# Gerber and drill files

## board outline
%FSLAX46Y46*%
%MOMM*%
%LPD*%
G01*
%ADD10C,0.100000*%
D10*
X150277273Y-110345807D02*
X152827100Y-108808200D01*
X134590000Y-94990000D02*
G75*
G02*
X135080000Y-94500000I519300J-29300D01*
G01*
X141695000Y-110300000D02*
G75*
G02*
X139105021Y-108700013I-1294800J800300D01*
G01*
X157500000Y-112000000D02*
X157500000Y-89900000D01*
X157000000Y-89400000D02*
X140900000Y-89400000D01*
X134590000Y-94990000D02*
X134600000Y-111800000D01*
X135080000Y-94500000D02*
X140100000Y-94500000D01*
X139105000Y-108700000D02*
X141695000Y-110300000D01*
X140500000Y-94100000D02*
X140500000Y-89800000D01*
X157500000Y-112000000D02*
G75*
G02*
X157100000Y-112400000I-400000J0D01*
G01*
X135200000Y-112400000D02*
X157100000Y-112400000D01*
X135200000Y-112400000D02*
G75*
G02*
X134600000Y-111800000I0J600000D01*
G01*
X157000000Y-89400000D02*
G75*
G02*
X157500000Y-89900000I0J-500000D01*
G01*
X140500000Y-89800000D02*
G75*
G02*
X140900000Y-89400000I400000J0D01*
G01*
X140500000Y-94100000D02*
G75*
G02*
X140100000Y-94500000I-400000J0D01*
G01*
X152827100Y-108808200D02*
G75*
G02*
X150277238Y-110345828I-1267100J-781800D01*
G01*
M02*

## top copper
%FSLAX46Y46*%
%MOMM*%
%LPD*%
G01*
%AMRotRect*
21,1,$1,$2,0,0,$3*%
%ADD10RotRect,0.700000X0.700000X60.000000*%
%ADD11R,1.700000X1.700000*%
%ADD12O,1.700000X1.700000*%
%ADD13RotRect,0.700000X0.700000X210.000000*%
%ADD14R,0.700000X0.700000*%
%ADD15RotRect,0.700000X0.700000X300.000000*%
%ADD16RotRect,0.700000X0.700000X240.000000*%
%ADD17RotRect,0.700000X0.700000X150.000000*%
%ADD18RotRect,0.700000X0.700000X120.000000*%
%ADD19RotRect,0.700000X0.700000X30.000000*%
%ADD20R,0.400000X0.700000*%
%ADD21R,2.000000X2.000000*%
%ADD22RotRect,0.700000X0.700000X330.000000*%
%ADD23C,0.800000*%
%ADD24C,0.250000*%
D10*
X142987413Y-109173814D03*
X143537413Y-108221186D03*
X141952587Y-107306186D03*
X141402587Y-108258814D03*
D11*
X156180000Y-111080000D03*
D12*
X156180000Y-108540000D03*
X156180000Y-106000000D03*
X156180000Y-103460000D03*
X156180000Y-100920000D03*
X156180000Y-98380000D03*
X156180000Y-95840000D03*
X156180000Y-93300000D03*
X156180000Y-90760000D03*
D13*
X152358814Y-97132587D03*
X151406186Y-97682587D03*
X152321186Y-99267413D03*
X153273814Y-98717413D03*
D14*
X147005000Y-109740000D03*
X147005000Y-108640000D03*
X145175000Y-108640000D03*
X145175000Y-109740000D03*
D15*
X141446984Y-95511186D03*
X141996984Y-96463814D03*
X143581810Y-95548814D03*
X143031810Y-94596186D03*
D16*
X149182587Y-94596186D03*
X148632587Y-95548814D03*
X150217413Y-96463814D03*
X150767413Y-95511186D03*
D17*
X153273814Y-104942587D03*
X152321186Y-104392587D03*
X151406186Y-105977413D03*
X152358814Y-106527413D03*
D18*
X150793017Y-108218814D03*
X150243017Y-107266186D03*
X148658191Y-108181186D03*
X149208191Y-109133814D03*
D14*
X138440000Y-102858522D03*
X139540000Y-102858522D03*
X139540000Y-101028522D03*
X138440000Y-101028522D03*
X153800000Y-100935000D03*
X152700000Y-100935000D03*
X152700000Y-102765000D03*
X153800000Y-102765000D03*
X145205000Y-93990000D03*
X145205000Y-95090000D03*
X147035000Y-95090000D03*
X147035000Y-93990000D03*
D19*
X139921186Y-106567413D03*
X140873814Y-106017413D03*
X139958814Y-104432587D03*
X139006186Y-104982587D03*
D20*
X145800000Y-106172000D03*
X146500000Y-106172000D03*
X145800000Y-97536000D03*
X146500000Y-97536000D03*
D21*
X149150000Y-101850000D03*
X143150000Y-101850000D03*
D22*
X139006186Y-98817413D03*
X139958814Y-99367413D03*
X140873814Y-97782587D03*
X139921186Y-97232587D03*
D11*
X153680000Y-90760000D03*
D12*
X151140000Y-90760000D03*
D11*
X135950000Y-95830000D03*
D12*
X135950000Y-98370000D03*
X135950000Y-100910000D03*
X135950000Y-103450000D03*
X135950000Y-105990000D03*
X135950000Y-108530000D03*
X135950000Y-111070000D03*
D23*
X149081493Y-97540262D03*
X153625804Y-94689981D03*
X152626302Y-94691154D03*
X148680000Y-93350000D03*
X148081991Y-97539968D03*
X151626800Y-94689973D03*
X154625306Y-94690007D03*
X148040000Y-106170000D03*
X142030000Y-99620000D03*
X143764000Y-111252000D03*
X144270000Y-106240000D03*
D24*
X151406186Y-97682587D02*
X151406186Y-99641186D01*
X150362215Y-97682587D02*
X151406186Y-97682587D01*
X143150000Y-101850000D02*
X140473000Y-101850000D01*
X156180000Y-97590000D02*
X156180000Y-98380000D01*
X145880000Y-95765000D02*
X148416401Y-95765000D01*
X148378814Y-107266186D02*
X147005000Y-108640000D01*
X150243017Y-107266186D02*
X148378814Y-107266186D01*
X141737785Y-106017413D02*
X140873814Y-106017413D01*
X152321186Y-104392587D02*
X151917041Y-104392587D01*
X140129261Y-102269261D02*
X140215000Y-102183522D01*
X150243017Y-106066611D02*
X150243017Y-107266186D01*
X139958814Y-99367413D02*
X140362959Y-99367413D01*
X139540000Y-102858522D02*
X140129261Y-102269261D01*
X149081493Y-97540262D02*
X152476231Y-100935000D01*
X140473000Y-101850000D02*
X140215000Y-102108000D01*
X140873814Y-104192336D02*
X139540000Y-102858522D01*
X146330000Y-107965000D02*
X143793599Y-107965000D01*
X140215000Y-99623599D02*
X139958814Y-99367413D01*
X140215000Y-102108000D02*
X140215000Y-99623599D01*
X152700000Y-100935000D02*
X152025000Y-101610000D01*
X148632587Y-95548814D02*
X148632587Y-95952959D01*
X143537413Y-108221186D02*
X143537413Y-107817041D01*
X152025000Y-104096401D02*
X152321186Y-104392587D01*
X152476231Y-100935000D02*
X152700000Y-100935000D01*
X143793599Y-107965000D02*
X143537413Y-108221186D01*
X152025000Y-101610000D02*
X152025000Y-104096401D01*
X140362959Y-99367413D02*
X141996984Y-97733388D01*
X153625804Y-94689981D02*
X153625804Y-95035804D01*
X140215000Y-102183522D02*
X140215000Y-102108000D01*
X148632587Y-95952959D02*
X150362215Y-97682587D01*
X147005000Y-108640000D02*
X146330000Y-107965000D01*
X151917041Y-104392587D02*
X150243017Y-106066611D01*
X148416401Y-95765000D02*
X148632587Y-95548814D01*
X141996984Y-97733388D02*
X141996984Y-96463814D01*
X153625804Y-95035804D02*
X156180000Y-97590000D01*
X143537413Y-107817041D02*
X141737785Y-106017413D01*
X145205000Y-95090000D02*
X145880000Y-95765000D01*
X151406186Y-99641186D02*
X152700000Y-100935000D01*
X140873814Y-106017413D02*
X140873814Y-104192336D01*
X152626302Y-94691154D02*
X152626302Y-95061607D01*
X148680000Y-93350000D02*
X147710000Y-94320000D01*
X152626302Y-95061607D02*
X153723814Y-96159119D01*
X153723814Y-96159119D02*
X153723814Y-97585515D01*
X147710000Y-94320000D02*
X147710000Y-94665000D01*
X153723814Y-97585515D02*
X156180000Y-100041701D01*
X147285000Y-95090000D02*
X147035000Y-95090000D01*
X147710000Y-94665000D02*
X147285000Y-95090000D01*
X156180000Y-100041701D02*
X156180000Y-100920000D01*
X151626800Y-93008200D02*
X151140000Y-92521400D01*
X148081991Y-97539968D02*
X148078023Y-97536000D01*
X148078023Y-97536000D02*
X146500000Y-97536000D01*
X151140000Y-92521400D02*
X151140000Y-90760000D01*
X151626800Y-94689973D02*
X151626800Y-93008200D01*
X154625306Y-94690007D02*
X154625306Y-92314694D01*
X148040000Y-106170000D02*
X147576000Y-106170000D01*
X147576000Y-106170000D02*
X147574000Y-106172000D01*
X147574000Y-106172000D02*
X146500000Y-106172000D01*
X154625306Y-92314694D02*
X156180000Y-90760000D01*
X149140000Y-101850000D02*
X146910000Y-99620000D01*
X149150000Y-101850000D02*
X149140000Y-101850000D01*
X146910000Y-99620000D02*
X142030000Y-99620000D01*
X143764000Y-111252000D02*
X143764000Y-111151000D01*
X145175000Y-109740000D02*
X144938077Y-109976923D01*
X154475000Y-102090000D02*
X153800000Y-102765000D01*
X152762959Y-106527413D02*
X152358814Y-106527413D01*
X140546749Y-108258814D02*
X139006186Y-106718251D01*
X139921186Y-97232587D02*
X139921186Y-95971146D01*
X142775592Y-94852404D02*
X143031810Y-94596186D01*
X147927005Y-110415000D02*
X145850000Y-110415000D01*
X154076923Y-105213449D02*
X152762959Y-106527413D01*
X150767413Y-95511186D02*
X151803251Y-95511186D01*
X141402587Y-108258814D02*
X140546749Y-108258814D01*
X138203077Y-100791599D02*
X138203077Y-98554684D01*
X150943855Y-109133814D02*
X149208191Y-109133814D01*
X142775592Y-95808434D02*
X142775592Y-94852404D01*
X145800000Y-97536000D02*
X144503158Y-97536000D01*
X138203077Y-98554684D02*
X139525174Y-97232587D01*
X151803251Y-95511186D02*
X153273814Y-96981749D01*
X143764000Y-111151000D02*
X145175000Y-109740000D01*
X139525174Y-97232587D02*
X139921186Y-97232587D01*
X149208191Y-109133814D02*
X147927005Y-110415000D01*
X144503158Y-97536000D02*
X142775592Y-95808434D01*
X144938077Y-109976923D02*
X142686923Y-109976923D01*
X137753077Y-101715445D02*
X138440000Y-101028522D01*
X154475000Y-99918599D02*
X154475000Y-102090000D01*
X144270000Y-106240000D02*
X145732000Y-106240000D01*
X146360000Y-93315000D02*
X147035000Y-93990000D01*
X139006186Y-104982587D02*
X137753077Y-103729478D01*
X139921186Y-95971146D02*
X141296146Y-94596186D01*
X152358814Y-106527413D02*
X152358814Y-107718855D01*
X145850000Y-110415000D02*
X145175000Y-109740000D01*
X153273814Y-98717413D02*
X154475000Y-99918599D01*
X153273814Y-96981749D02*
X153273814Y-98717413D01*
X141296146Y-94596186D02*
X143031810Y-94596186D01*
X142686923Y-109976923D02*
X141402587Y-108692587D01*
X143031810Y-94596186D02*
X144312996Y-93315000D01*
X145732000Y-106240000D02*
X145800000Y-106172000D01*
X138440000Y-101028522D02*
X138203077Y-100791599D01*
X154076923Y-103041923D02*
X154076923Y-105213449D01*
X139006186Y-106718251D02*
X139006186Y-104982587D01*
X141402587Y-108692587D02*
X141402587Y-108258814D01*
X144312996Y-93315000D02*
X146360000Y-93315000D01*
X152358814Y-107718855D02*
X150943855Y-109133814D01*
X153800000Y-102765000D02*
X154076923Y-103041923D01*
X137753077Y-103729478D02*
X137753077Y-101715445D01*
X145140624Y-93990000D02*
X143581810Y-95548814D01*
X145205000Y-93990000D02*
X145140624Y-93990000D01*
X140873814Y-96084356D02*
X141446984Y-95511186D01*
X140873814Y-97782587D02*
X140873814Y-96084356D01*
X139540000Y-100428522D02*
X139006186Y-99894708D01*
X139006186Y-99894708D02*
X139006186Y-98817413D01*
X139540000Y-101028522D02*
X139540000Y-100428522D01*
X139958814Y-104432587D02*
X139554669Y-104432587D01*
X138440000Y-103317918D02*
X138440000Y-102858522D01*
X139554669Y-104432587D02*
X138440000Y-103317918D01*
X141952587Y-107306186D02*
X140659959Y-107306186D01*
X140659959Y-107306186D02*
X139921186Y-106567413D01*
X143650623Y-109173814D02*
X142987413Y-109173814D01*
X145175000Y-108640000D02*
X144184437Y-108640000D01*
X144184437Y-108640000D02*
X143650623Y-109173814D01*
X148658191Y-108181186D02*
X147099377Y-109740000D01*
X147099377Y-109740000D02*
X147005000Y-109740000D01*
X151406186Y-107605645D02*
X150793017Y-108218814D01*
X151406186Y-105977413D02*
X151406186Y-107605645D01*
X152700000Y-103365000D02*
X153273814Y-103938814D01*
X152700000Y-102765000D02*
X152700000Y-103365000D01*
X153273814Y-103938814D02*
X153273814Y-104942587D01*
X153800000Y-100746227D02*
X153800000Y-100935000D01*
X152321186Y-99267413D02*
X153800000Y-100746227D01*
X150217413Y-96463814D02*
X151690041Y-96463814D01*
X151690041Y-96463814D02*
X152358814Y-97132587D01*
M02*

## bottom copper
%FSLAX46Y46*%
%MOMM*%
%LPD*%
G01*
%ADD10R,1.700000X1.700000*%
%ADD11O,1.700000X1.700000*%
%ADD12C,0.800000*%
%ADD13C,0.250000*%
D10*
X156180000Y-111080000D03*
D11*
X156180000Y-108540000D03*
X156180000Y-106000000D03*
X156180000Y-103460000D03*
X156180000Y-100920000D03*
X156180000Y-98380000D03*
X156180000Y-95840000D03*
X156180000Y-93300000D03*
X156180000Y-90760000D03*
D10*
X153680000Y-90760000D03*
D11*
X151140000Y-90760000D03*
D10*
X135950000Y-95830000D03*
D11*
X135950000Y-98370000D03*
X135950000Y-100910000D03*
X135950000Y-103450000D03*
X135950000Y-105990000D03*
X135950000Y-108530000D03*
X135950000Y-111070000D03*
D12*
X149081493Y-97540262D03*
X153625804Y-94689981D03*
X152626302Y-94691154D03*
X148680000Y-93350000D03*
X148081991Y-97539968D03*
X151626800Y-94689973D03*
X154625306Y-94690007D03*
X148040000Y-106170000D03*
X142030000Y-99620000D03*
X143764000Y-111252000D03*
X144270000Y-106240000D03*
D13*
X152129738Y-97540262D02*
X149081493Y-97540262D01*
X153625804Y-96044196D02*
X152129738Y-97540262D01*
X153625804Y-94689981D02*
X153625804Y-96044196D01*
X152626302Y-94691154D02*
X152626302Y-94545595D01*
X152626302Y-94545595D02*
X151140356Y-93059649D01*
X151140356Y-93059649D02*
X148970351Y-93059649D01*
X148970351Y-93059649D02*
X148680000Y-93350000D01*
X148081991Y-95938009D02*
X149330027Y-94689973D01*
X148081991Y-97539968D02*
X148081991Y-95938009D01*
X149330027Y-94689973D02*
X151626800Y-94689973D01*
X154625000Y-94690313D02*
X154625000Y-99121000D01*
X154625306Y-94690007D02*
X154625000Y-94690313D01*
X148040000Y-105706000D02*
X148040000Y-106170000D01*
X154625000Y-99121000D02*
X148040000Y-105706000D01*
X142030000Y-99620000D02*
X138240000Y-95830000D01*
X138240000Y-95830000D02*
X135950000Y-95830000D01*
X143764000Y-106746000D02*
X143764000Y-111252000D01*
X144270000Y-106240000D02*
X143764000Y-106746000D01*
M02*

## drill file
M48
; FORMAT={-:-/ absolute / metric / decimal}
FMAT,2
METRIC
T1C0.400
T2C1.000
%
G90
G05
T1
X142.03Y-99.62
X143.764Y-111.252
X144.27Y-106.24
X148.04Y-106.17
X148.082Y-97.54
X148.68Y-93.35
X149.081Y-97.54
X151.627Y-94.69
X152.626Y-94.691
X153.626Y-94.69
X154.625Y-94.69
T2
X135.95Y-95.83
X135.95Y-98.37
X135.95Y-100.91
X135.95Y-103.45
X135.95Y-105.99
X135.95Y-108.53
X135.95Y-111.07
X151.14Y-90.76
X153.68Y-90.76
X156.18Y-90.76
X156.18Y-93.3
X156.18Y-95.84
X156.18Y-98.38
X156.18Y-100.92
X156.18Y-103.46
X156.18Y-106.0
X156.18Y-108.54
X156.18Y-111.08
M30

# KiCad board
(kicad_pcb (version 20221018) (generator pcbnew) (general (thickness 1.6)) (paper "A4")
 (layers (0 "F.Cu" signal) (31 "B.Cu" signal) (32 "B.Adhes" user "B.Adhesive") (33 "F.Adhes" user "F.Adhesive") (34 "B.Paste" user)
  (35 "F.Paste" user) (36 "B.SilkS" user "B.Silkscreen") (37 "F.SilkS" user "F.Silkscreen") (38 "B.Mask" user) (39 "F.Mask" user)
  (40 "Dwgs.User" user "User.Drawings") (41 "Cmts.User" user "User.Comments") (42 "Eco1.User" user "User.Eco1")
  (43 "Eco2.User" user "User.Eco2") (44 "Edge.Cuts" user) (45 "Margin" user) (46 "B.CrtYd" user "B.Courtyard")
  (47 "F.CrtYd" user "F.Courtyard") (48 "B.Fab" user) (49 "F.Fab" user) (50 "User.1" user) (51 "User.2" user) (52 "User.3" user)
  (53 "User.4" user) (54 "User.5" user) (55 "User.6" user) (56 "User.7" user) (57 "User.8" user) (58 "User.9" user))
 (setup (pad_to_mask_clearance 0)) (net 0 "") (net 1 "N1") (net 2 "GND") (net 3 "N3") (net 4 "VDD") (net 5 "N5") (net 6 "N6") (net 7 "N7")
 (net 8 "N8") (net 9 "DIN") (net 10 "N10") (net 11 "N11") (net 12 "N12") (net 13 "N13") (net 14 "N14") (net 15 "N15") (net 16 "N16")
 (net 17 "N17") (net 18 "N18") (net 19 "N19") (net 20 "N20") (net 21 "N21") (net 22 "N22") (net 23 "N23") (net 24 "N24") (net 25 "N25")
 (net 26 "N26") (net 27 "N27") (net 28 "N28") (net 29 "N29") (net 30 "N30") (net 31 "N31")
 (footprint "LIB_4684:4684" (layer "F.Cu") (at 142.47 108.24 -30)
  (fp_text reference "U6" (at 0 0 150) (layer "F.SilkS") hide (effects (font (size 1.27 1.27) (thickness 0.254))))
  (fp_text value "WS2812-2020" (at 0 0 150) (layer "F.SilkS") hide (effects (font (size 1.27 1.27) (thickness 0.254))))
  (pad "1" smd rect (at 0.915 0.55 60) (size 0.7 0.7) (layers "F.Cu" "F.Paste" "F.Mask") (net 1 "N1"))
  (pad "2" smd rect (at 0.915 -0.55 60) (size 0.7 0.7) (layers "F.Cu" "F.Paste" "F.Mask") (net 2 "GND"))
  (pad "3" smd rect (at -0.915 -0.55 60) (size 0.7 0.7) (layers "F.Cu" "F.Paste" "F.Mask") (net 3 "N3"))
  (pad "4" smd rect (at -0.915 0.55 60) (size 0.7 0.7) (layers "F.Cu" "F.Paste" "F.Mask") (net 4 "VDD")))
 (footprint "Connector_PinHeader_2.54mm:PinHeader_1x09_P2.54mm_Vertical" (layer "F.Cu") (at 156.18 111.08 180)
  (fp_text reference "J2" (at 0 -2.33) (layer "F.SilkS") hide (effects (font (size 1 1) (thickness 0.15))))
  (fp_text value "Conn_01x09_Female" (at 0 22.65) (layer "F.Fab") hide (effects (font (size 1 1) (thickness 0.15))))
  (pad "1" thru_hole rect (at 0 0 180) (size 1.7 1.7) (drill 1) (layers "*.Cu" "*.Mask") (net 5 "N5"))
  (pad "2" thru_hole oval (at 0 2.54 180) (size 1.7 1.7) (drill 1) (layers "*.Cu" "*.Mask") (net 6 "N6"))
  (pad "3" thru_hole oval (at 0 5.08 180) (size 1.7 1.7) (drill 1) (layers "*.Cu" "*.Mask") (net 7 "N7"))
  (pad "4" thru_hole oval (at 0 7.62 180) (size 1.7 1.7) (drill 1) (layers "*.Cu" "*.Mask") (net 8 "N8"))
  (pad "5" thru_hole oval (at 0 10.16 180) (size 1.7 1.7) (drill 1) (layers "*.Cu" "*.Mask") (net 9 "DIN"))
  (pad "6" thru_hole oval (at 0 12.7 180) (size 1.7 1.7) (drill 1) (layers "*.Cu" "*.Mask") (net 2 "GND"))
  (pad "7" thru_hole oval (at 0 15.24 180) (size 1.7 1.7) (drill 1) (layers "*.Cu" "*.Mask") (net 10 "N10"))
  (pad "8" thru_hole oval (at 0 17.78 180) (size 1.7 1.7) (drill 1) (layers "*.Cu" "*.Mask") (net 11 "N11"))
  (pad "9" thru_hole oval (at 0 20.32 180) (size 1.7 1.7) (drill 1) (layers "*.Cu" "*.Mask") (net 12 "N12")))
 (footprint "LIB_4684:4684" (layer "F.Cu") (at 152.34 98.2 120)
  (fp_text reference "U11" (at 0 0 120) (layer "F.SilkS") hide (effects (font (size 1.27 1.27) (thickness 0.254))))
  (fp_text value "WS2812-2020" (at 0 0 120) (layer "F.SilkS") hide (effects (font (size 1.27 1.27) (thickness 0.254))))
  (pad "1" smd rect (at 0.915 0.55 210) (size 0.7 0.7) (layers "F.Cu" "F.Paste" "F.Mask") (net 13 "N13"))
  (pad "2" smd rect (at 0.915 -0.55 210) (size 0.7 0.7) (layers "F.Cu" "F.Paste" "F.Mask") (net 2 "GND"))
  (pad "3" smd rect (at -0.915 -0.55 210) (size 0.7 0.7) (layers "F.Cu" "F.Paste" "F.Mask") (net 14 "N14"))
  (pad "4" smd rect (at -0.915 0.55 210) (size 0.7 0.7) (layers "F.Cu" "F.Paste" "F.Mask") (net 4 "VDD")))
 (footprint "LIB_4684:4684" (layer "F.Cu") (at 146.09 109.19)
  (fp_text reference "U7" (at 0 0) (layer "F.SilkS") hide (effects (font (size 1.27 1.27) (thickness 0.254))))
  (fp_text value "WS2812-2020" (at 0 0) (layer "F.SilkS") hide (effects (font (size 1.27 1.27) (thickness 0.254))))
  (pad "1" smd rect (at 0.915 0.55 90) (size 0.7 0.7) (layers "F.Cu" "F.Paste" "F.Mask") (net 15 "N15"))
  (pad "2" smd rect (at 0.915 -0.55 90) (size 0.7 0.7) (layers "F.Cu" "F.Paste" "F.Mask") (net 2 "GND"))
  (pad "3" smd rect (at -0.915 -0.55 90) (size 0.7 0.7) (layers "F.Cu" "F.Paste" "F.Mask") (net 1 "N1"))
  (pad "4" smd rect (at -0.915 0.55 90) (size 0.7 0.7) (layers "F.Cu" "F.Paste" "F.Mask") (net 4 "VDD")))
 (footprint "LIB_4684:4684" (layer "F.Cu") (at 142.514397 95.53 -150)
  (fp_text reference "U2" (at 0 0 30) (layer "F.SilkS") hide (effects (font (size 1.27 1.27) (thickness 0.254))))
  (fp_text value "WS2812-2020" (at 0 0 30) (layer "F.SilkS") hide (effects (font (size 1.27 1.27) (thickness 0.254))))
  (pad "1" smd rect (at 0.915 0.55 300) (size 0.7 0.7) (layers "F.Cu" "F.Paste" "F.Mask") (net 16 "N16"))
  (pad "2" smd rect (at 0.915 -0.55 300) (size 0.7 0.7) (layers "F.Cu" "F.Paste" "F.Mask") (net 2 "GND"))
  (pad "3" smd rect (at -0.915 -0.55 300) (size 0.7 0.7) (layers "F.Cu" "F.Paste" "F.Mask") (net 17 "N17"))
  (pad "4" smd rect (at -0.915 0.55 300) (size 0.7 0.7) (layers "F.Cu" "F.Paste" "F.Mask") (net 4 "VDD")))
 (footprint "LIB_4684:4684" (layer "F.Cu") (at 149.7 95.53 150)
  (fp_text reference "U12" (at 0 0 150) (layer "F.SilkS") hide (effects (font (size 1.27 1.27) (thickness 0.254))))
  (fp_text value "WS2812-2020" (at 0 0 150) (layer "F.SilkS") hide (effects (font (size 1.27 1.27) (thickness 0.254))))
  (pad "1" smd rect (at 0.915 0.55 240) (size 0.7 0.7) (layers "F.Cu" "F.Paste" "F.Mask") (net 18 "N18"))
  (pad "2" smd rect (at 0.915 -0.55 240) (size 0.7 0.7) (layers "F.Cu" "F.Paste" "F.Mask") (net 2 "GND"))
  (pad "3" smd rect (at -0.915 -0.55 240) (size 0.7 0.7) (layers "F.Cu" "F.Paste" "F.Mask") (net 13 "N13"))
  (pad "4" smd rect (at -0.915 0.55 240) (size 0.7 0.7) (layers "F.Cu" "F.Paste" "F.Mask") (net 4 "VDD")))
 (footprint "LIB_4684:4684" (layer "F.Cu") (at 152.34 105.46 60)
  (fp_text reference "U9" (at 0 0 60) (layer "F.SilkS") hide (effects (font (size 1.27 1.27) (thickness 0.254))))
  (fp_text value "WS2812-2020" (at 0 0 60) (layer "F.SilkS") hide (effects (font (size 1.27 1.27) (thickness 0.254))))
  (pad "1" smd rect (at 0.915 0.55 150) (size 0.7 0.7) (layers "F.Cu" "F.Paste" "F.Mask") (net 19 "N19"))
  (pad "2" smd rect (at 0.915 -0.55 150) (size 0.7 0.7) (layers "F.Cu" "F.Paste" "F.Mask") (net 2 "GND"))
  (pad "3" smd rect (at -0.915 -0.55 150) (size 0.7 0.7) (layers "F.Cu" "F.Paste" "F.Mask") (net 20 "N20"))
  (pad "4" smd rect (at -0.915 0.55 150) (size 0.7 0.7) (layers "F.Cu" "F.Paste" "F.Mask") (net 4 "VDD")))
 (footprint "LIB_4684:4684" (layer "F.Cu") (at 149.725604 108.2 30)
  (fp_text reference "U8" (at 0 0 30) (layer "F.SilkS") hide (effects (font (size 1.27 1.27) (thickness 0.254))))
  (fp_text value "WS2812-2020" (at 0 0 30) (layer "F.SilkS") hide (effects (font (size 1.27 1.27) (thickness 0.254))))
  (pad "1" smd rect (at 0.915 0.55 120) (size 0.7 0.7) (layers "F.Cu" "F.Paste" "F.Mask") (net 20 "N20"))
  (pad "2" smd rect (at 0.915 -0.55 120) (size 0.7 0.7) (layers "F.Cu" "F.Paste" "F.Mask") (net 2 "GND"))
  (pad "3" smd rect (at -0.915 -0.55 120) (size 0.7 0.7) (layers "F.Cu" "F.Paste" "F.Mask") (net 15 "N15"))
  (pad "4" smd rect (at -0.915 0.55 120) (size 0.7 0.7) (layers "F.Cu" "F.Paste" "F.Mask") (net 4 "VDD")))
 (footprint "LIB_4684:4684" (layer "F.Cu") (at 138.99 101.943522 -90)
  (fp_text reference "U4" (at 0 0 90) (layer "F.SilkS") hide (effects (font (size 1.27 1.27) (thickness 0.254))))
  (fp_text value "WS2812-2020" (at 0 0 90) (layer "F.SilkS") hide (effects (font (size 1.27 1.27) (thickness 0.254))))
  (pad "1" smd rect (at 0.915 0.55) (size 0.7 0.7) (layers "F.Cu" "F.Paste" "F.Mask") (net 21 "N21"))
  (pad "2" smd rect (at 0.915 -0.55) (size 0.7 0.7) (layers "F.Cu" "F.Paste" "F.Mask") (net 2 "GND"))
  (pad "3" smd rect (at -0.915 -0.55) (size 0.7 0.7) (layers "F.Cu" "F.Paste" "F.Mask") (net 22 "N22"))
  (pad "4" smd rect (at -0.915 0.55) (size 0.7 0.7) (layers "F.Cu" "F.Paste" "F.Mask") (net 4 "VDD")))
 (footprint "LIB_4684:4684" (layer "F.Cu") (at 153.25 101.85 90)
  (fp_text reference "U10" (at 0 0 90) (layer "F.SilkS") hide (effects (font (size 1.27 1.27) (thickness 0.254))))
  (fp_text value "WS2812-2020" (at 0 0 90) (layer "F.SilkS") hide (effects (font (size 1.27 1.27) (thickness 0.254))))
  (pad "1" smd rect (at 0.915 0.55 180) (size 0.7 0.7) (layers "F.Cu" "F.Paste" "F.Mask") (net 14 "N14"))
  (pad "2" smd rect (at 0.915 -0.55 180) (size 0.7 0.7) (layers "F.Cu" "F.Paste" "F.Mask") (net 2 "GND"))
  (pad "3" smd rect (at -0.915 -0.55 180) (size 0.7 0.7) (layers "F.Cu" "F.Paste" "F.Mask") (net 19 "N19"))
  (pad "4" smd rect (at -0.915 0.55 180) (size 0.7 0.7) (layers "F.Cu" "F.Paste" "F.Mask") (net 4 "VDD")))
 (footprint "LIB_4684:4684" (layer "F.Cu") (at 146.12 94.54 180)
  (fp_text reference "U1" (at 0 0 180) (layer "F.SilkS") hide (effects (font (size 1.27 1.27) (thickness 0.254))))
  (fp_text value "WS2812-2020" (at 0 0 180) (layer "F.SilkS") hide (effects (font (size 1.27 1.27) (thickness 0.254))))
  (pad "1" smd rect (at 0.915 0.55 270) (size 0.7 0.7) (layers "F.Cu" "F.Paste" "F.Mask") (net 17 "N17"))
  (pad "2" smd rect (at 0.915 -0.55 270) (size 0.7 0.7) (layers "F.Cu" "F.Paste" "F.Mask") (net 2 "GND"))
  (pad "3" smd rect (at -0.915 -0.55 270) (size 0.7 0.7) (layers "F.Cu" "F.Paste" "F.Mask") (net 9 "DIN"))
  (pad "4" smd rect (at -0.915 0.55 270) (size 0.7 0.7) (layers "F.Cu" "F.Paste" "F.Mask") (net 4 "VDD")))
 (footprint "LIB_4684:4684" (layer "F.Cu") (at 139.94 105.5 -60)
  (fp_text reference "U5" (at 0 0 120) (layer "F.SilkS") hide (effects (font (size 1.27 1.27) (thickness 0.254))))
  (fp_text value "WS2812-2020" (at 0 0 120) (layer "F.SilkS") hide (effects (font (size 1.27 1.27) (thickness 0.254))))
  (pad "1" smd rect (at 0.915 0.55 30) (size 0.7 0.7) (layers "F.Cu" "F.Paste" "F.Mask") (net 3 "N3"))
  (pad "2" smd rect (at 0.915 -0.55 30) (size 0.7 0.7) (layers "F.Cu" "F.Paste" "F.Mask") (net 2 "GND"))
  (pad "3" smd rect (at -0.915 -0.55 30) (size 0.7 0.7) (layers "F.Cu" "F.Paste" "F.Mask") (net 21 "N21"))
  (pad "4" smd rect (at -0.915 0.55 30) (size 0.7 0.7) (layers "F.Cu" "F.Paste" "F.Mask") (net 4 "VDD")))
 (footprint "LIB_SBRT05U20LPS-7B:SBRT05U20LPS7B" (layer "F.Cu") (at 146.15 106.172)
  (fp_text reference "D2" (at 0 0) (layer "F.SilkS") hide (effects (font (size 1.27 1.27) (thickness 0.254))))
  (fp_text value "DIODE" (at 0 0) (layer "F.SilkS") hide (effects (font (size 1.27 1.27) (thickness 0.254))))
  (pad "1" smd rect (at -0.35 0) (size 0.4 0.7) (layers "F.Cu" "F.Paste" "F.Mask") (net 4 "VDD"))
  (pad "2" smd rect (at 0.35 0) (size 0.4 0.7) (layers "F.Cu" "F.Paste" "F.Mask") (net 12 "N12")))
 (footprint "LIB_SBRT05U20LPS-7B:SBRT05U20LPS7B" (layer "F.Cu") (at 146.15 97.536)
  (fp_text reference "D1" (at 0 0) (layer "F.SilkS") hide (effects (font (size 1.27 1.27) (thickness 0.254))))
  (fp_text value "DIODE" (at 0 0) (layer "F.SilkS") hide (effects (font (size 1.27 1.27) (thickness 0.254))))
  (pad "1" smd rect (at -0.35 0) (size 0.4 0.7) (layers "F.Cu" "F.Paste" "F.Mask") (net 4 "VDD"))
  (pad "2" smd rect (at 0.35 0) (size 0.4 0.7) (layers "F.Cu" "F.Paste" "F.Mask") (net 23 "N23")))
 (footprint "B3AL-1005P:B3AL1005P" (layer "F.Cu") (at 146.15 101.85)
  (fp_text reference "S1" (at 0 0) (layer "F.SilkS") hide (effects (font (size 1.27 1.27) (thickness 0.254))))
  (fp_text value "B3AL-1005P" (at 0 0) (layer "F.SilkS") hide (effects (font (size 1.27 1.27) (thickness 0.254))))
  (pad "1" smd rect (at 3 0 90) (size 2 2) (layers "F.Cu" "F.Paste" "F.Mask") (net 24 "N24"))
  (pad "2" smd rect (at -3 0 90) (size 2 2) (layers "F.Cu" "F.Paste" "F.Mask") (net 2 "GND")))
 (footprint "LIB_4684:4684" (layer "F.Cu") (at 139.94 98.3 -120)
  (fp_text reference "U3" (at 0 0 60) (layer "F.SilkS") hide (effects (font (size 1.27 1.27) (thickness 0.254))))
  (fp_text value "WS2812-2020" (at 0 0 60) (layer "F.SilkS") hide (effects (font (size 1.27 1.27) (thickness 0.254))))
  (pad "1" smd rect (at 0.915 0.55 330) (size 0.7 0.7) (layers "F.Cu" "F.Paste" "F.Mask") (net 22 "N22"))
  (pad "2" smd rect (at 0.915 -0.55 330) (size 0.7 0.7) (layers "F.Cu" "F.Paste" "F.Mask") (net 2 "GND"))
  (pad "3" smd rect (at -0.915 -0.55 330) (size 0.7 0.7) (layers "F.Cu" "F.Paste" "F.Mask") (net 16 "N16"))
  (pad "4" smd rect (at -0.915 0.55 330) (size 0.7 0.7) (layers "F.Cu" "F.Paste" "F.Mask") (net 4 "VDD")))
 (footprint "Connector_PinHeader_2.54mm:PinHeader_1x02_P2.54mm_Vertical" (layer "F.Cu") (at 153.68 90.76 -90)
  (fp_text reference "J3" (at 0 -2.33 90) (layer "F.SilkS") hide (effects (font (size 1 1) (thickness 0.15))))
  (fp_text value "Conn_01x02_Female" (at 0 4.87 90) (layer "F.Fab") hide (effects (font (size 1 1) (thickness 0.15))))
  (pad "1" thru_hole rect (at 0 0 270) (size 1.7 1.7) (drill 1) (layers "*.Cu" "*.Mask") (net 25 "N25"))
  (pad "2" thru_hole oval (at 0 2.54 270) (size 1.7 1.7) (drill 1) (layers "*.Cu" "*.Mask") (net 23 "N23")))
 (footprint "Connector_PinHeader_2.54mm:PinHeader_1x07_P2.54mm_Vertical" (layer "F.Cu") (at 135.95 95.83)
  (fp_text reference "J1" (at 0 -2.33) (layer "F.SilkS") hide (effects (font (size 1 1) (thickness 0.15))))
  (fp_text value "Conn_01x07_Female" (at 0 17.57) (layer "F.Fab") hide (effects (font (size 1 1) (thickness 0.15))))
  (pad "1" thru_hole rect (at 0 0) (size 1.7 1.7) (drill 1) (layers "*.Cu" "*.Mask") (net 24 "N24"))
  (pad "2" thru_hole oval (at 0 2.54) (size 1.7 1.7) (drill 1) (layers "*.Cu" "*.Mask") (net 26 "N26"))
  (pad "3" thru_hole oval (at 0 5.08) (size 1.7 1.7) (drill 1) (layers "*.Cu" "*.Mask") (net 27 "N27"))
  (pad "4" thru_hole oval (at 0 7.62) (size 1.7 1.7) (drill 1) (layers "*.Cu" "*.Mask") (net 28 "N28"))
  (pad "5" thru_hole oval (at 0 10.16) (size 1.7 1.7) (drill 1) (layers "*.Cu" "*.Mask") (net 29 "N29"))
  (pad "6" thru_hole oval (at 0 12.7) (size 1.7 1.7) (drill 1) (layers "*.Cu" "*.Mask") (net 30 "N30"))
  (pad "7" thru_hole oval (at 0 15.24) (size 1.7 1.7) (drill 1) (layers "*.Cu" "*.Mask") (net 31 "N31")))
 (gr_line (start 150.277273 110.345807) (end 152.8271 108.8082) (stroke (width 0.1) (type solid)) (layer "Edge.Cuts"))
 (gr_arc (start 134.59 94.99) (mid 134.741518 94.651518) (end 135.08 94.5) (stroke (width 0.1) (type solid)) (layer "Edge.Cuts"))
 (gr_arc (start 141.695 110.3) (mid 139.600179 110.794634) (end 139.105 108.7) (stroke (width 0.1) (type solid)) (layer "Edge.Cuts"))
 (gr_line (start 157.5 112) (end 157.5 89.9) (stroke (width 0.1) (type solid)) (layer "Edge.Cuts"))
 (gr_line (start 157 89.4) (end 140.9 89.4) (stroke (width 0.1) (type solid)) (layer "Edge.Cuts"))
 (gr_line (start 134.59 94.99) (end 134.6 111.8) (stroke (width 0.1) (type solid)) (layer "Edge.Cuts"))
 (gr_line (start 135.08 94.5) (end 140.1 94.5) (stroke (width 0.1) (type solid)) (layer "Edge.Cuts"))
 (gr_line (start 139.105 108.7) (end 141.695 110.3) (stroke (width 0.1) (type solid)) (layer "Edge.Cuts"))
 (gr_line (start 140.5 94.1) (end 140.5 89.8) (stroke (width 0.1) (type solid)) (layer "Edge.Cuts"))
 (gr_arc (start 157.5 112) (mid 157.382843 112.282843) (end 157.1 112.4) (stroke (width 0.1) (type solid)) (layer "Edge.Cuts"))
 (gr_line (start 135.2 112.4) (end 157.1 112.4) (stroke (width 0.1) (type solid)) (layer "Edge.Cuts"))
 (gr_arc (start 135.2 112.4) (mid 134.775736 112.224264) (end 134.6 111.8) (stroke (width 0.1) (type solid)) (layer "Edge.Cuts"))
 (gr_arc (start 157 89.4) (mid 157.353553 89.546447) (end 157.5 89.9) (stroke (width 0.1) (type solid)) (layer "Edge.Cuts"))
 (gr_arc (start 140.5 89.8) (mid 140.617157 89.517157) (end 140.9 89.4) (stroke (width 0.1) (type solid)) (layer "Edge.Cuts"))
 (gr_arc (start 140.5 94.1) (mid 140.382843 94.382843) (end 140.1 94.5) (stroke (width 0.1) (type solid)) (layer "Edge.Cuts"))
 (gr_arc (start 152.8271 108.8082) (mid 152.328854 110.864997) (end 150.277273 110.345807) (stroke (width 0.1) (type solid))
  (layer "Edge.Cuts"))
 (segment (start 151.406186 97.682587) (end 151.406186 99.641186) (width 0.25) (layer "F.Cu") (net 2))
 (segment (start 150.362215 97.682587) (end 151.406186 97.682587) (width 0.25) (layer "F.Cu") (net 2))
 (segment (start 143.15 101.85) (end 140.473 101.85) (width 0.25) (layer "F.Cu") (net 2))
 (segment (start 156.18 97.59) (end 156.18 98.38) (width 0.25) (layer "F.Cu") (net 2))
 (segment (start 145.88 95.765) (end 148.416401 95.765) (width 0.25) (layer "F.Cu") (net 2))
 (segment (start 148.378814 107.266186) (end 147.005 108.64) (width 0.25) (layer "F.Cu") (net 2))
 (segment (start 150.243017 107.266186) (end 148.378814 107.266186) (width 0.25) (layer "F.Cu") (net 2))
 (segment (start 141.737785 106.017413) (end 140.873814 106.017413) (width 0.25) (layer "F.Cu") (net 2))
 (segment (start 152.321186 104.392587) (end 151.917041 104.392587) (width 0.25) (layer "F.Cu") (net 2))
 (segment (start 140.129261 102.269261) (end 140.215 102.183522) (width 0.25) (layer "F.Cu") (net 2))
 (segment (start 150.243017 106.066611) (end 150.243017 107.266186) (width 0.25) (layer "F.Cu") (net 2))
 (segment (start 139.958814 99.367413) (end 140.362959 99.367413) (width 0.25) (layer "F.Cu") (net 2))
 (segment (start 139.54 102.858522) (end 140.129261 102.269261) (width 0.25) (layer "F.Cu") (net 2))
 (segment (start 149.081493 97.540262) (end 152.476231 100.935) (width 0.25) (layer "F.Cu") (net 2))
 (segment (start 140.473 101.85) (end 140.215 102.108) (width 0.25) (layer "F.Cu") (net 2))
 (segment (start 140.873814 104.192336) (end 139.54 102.858522) (width 0.25) (layer "F.Cu") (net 2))
 (segment (start 146.33 107.965) (end 143.793599 107.965) (width 0.25) (layer "F.Cu") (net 2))
 (segment (start 140.215 99.623599) (end 139.958814 99.367413) (width 0.25) (layer "F.Cu") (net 2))
 (segment (start 140.215 102.108) (end 140.215 99.623599) (width 0.25) (layer "F.Cu") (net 2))
 (segment (start 152.7 100.935) (end 152.025 101.61) (width 0.25) (layer "F.Cu") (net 2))
 (segment (start 148.632587 95.548814) (end 148.632587 95.952959) (width 0.25) (layer "F.Cu") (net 2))
 (segment (start 143.537413 108.221186) (end 143.537413 107.817041) (width 0.25) (layer "F.Cu") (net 2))
 (segment (start 152.025 104.096401) (end 152.321186 104.392587) (width 0.25) (layer "F.Cu") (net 2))
 (segment (start 152.476231 100.935) (end 152.7 100.935) (width 0.25) (layer "F.Cu") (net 2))
 (segment (start 143.793599 107.965) (end 143.537413 108.221186) (width 0.25) (layer "F.Cu") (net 2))
 (segment (start 152.025 101.61) (end 152.025 104.096401) (width 0.25) (layer "F.Cu") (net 2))
 (segment (start 140.362959 99.367413) (end 141.996984 97.733388) (width 0.25) (layer "F.Cu") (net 2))
 (segment (start 153.625804 94.689981) (end 153.625804 95.035804) (width 0.25) (layer "F.Cu") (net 2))
 (segment (start 140.215 102.183522) (end 140.215 102.108) (width 0.25) (layer "F.Cu") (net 2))
 (segment (start 148.632587 95.952959) (end 150.362215 97.682587) (width 0.25) (layer "F.Cu") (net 2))
 (segment (start 147.005 108.64) (end 146.33 107.965) (width 0.25) (layer "F.Cu") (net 2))
 (segment (start 151.917041 104.392587) (end 150.243017 106.066611) (width 0.25) (layer "F.Cu") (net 2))
 (segment (start 148.416401 95.765) (end 148.632587 95.548814) (width 0.25) (layer "F.Cu") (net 2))
 (segment (start 141.996984 97.733388) (end 141.996984 96.463814) (width 0.25) (layer "F.Cu") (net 2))
 (segment (start 153.625804 95.035804) (end 156.18 97.59) (width 0.25) (layer "F.Cu") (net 2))
 (segment (start 143.537413 107.817041) (end 141.737785 106.017413) (width 0.25) (layer "F.Cu") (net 2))
 (segment (start 145.205 95.09) (end 145.88 95.765) (width 0.25) (layer "F.Cu") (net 2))
 (segment (start 151.406186 99.641186) (end 152.7 100.935) (width 0.25) (layer "F.Cu") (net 2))
 (segment (start 140.873814 106.017413) (end 140.873814 104.192336) (width 0.25) (layer "F.Cu") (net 2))
 (via (at 149.081493 97.540262) (size 0.8) (drill 0.4) (layers "F.Cu" "B.Cu") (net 2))
 (via (at 153.625804 94.689981) (size 0.8) (drill 0.4) (layers "F.Cu" "B.Cu") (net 2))
 (segment (start 152.129738 97.540262) (end 149.081493 97.540262) (width 0.25) (layer "B.Cu") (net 2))
 (segment (start 153.625804 96.044196) (end 152.129738 97.540262) (width 0.25) (layer "B.Cu") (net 2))
 (segment (start 153.625804 94.689981) (end 153.625804 96.044196) (width 0.25) (layer "B.Cu") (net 2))
 (segment (start 152.626302 94.691154) (end 152.626302 95.061607) (width 0.25) (layer "F.Cu") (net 9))
 (segment (start 148.68 93.35) (end 147.71 94.32) (width 0.25) (layer "F.Cu") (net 9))
 (segment (start 152.626302 95.061607) (end 153.723814 96.159119) (width 0.25) (layer "F.Cu") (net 9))
 (segment (start 153.723814 96.159119) (end 153.723814 97.585515) (width 0.25) (layer "F.Cu") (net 9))
 (segment (start 147.71 94.32) (end 147.71 94.665) (width 0.25) (layer "F.Cu") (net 9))
 (segment (start 153.723814 97.585515) (end 156.18 100.041701) (width 0.25) (layer "F.Cu") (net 9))
 (segment (start 147.285 95.09) (end 147.035 95.09) (width 0.25) (layer "F.Cu") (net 9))
 (segment (start 147.71 94.665) (end 147.285 95.09) (width 0.25) (layer "F.Cu") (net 9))
 (segment (start 156.18 100.041701) (end 156.18 100.92) (width 0.25) (layer "F.Cu") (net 9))
 (via (at 152.626302 94.691154) (size 0.8) (drill 0.4) (layers "F.Cu" "B.Cu") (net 9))
 (via (at 148.68 93.35) (size 0.8) (drill 0.4) (layers "F.Cu" "B.Cu") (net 9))
 (segment (start 152.626302 94.691154) (end 152.626302 94.545595) (width 0.25) (layer "B.Cu") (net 9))
 (segment (start 152.626302 94.545595) (end 151.140356 93.059649) (width 0.25) (layer "B.Cu") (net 9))
 (segment (start 151.140356 93.059649) (end 148.970351 93.059649) (width 0.25) (layer "B.Cu") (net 9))
 (segment (start 148.970351 93.059649) (end 148.68 93.35) (width 0.25) (layer "B.Cu") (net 9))
 (segment (start 151.6268 93.0082) (end 151.14 92.5214) (width 0.25) (layer "F.Cu") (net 23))
 (segment (start 148.081991 97.539968) (end 148.078023 97.536) (width 0.25) (layer "F.Cu") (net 23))
 (segment (start 148.078023 97.536) (end 146.5 97.536) (width 0.25) (layer "F.Cu") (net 23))
 (segment (start 151.14 92.5214) (end 151.14 90.76) (width 0.25) (layer "F.Cu") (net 23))
 (segment (start 151.6268 94.689973) (end 151.6268 93.0082) (width 0.25) (layer "F.Cu") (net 23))
 (via (at 148.081991 97.539968) (size 0.8) (drill 0.4) (layers "F.Cu" "B.Cu") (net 23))
 (via (at 151.6268 94.689973) (size 0.8) (drill 0.4) (layers "F.Cu" "B.Cu") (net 23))
 (segment (start 148.081991 95.938009) (end 149.330027 94.689973) (width 0.25) (layer "B.Cu") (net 23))
 (segment (start 148.081991 97.539968) (end 148.081991 95.938009) (width 0.25) (layer "B.Cu") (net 23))
 (segment (start 149.330027 94.689973) (end 151.6268 94.689973) (width 0.25) (layer "B.Cu") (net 23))
 (segment (start 154.625306 94.690007) (end 154.625306 92.314694) (width 0.25) (layer "F.Cu") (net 12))
 (segment (start 148.04 106.17) (end 147.576 106.17) (width 0.25) (layer "F.Cu") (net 12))
 (segment (start 147.576 106.17) (end 147.574 106.172) (width 0.25) (layer "F.Cu") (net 12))
 (segment (start 147.574 106.172) (end 146.5 106.172) (width 0.25) (layer "F.Cu") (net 12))
 (segment (start 154.625306 92.314694) (end 156.18 90.76) (width 0.25) (layer "F.Cu") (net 12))
 (via (at 154.625306 94.690007) (size 0.8) (drill 0.4) (layers "F.Cu" "B.Cu") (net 12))
 (via (at 148.04 106.17) (size 0.8) (drill 0.4) (layers "F.Cu" "B.Cu") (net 12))
 (segment (start 154.625 94.690313) (end 154.625 99.121) (width 0.25) (layer "B.Cu") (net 12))
 (segment (start 154.625306 94.690007) (end 154.625 94.690313) (width 0.25) (layer "B.Cu") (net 12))
 (segment (start 148.04 105.706) (end 148.04 106.17) (width 0.25) (layer "B.Cu") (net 12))
 (segment (start 154.625 99.121) (end 148.04 105.706) (width 0.25) (layer "B.Cu") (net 12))
 (segment (start 149.14 101.85) (end 146.91 99.62) (width 0.25) (layer "F.Cu") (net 24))
 (segment (start 149.15 101.85) (end 149.14 101.85) (width 0.25) (layer "F.Cu") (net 24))
 (segment (start 146.91 99.62) (end 142.03 99.62) (width 0.25) (layer "F.Cu") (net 24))
 (via (at 142.03 99.62) (size 0.8) (drill 0.4) (layers "F.Cu" "B.Cu") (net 24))
 (segment (start 142.03 99.62) (end 138.24 95.83) (width 0.25) (layer "B.Cu") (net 24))
 (segment (start 138.24 95.83) (end 135.95 95.83) (width 0.25) (layer "B.Cu") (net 24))
 (segment (start 143.764 111.252) (end 143.764 111.151) (width 0.25) (layer "F.Cu") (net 4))
 (segment (start 145.175 109.74) (end 144.938077 109.976923) (width 0.25) (layer "F.Cu") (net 4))
 (segment (start 154.475 102.09) (end 153.8 102.765) (width 0.25) (layer "F.Cu") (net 4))
 (segment (start 152.762959 106.527413) (end 152.358814 106.527413) (width 0.25) (layer "F.Cu") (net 4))
 (segment (start 140.546749 108.258814) (end 139.006186 106.718251) (width 0.25) (layer "F.Cu") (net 4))
 (segment (start 139.921186 97.232587) (end 139.921186 95.971146) (width 0.25) (layer "F.Cu") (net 4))
 (segment (start 142.775592 94.852404) (end 143.03181 94.596186) (width 0.25) (layer "F.Cu") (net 4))
 (segment (start 147.927005 110.415) (end 145.85 110.415) (width 0.25) (layer "F.Cu") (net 4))
 (segment (start 154.076923 105.213449) (end 152.762959 106.527413) (width 0.25) (layer "F.Cu") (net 4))
 (segment (start 150.767413 95.511186) (end 151.803251 95.511186) (width 0.25) (layer "F.Cu") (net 4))
 (segment (start 141.402587 108.258814) (end 140.546749 108.258814) (width 0.25) (layer "F.Cu") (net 4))
 (segment (start 138.203077 100.791599) (end 138.203077 98.554684) (width 0.25) (layer "F.Cu") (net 4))
 (segment (start 150.943855 109.133814) (end 149.208191 109.133814) (width 0.25) (layer "F.Cu") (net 4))
 (segment (start 142.775592 95.808434) (end 142.775592 94.852404) (width 0.25) (layer "F.Cu") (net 4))
 (segment (start 145.8 97.536) (end 144.503158 97.536) (width 0.25) (layer "F.Cu") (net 4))
 (segment (start 138.203077 98.554684) (end 139.525174 97.232587) (width 0.25) (layer "F.Cu") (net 4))
 (segment (start 151.803251 95.511186) (end 153.273814 96.981749) (width 0.25) (layer "F.Cu") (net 4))
 (segment (start 143.764 111.151) (end 145.175 109.74) (width 0.25) (layer "F.Cu") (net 4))
 (segment (start 139.525174 97.232587) (end 139.921186 97.232587) (width 0.25) (layer "F.Cu") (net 4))
 (segment (start 149.208191 109.133814) (end 147.927005 110.415) (width 0.25) (layer "F.Cu") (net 4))
 (segment (start 144.503158 97.536) (end 142.775592 95.808434) (width 0.25) (layer "F.Cu") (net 4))
 (segment (start 144.938077 109.976923) (end 142.686923 109.976923) (width 0.25) (layer "F.Cu") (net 4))
 (segment (start 137.753077 101.715445) (end 138.44 101.028522) (width 0.25) (layer "F.Cu") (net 4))
 (segment (start 154.475 99.918599) (end 154.475 102.09) (width 0.25) (layer "F.Cu") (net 4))
 (segment (start 144.27 106.24) (end 145.732 106.24) (width 0.25) (layer "F.Cu") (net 4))
 (segment (start 146.36 93.315) (end 147.035 93.99) (width 0.25) (layer "F.Cu") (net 4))
 (segment (start 139.006186 104.982587) (end 137.753077 103.729478) (width 0.25) (layer "F.Cu") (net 4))
 (segment (start 139.921186 95.971146) (end 141.296146 94.596186) (width 0.25) (layer "F.Cu") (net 4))
 (segment (start 152.358814 106.527413) (end 152.358814 107.718855) (width 0.25) (layer "F.Cu") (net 4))
 (segment (start 145.85 110.415) (end 145.175 109.74) (width 0.25) (layer "F.Cu") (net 4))
 (segment (start 153.273814 98.717413) (end 154.475 99.918599) (width 0.25) (layer "F.Cu") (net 4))
 (segment (start 153.273814 96.981749) (end 153.273814 98.717413) (width 0.25) (layer "F.Cu") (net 4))
 (segment (start 141.296146 94.596186) (end 143.03181 94.596186) (width 0.25) (layer "F.Cu") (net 4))
 (segment (start 142.686923 109.976923) (end 141.402587 108.692587) (width 0.25) (layer "F.Cu") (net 4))
 (segment (start 143.03181 94.596186) (end 144.312996 93.315) (width 0.25) (layer "F.Cu") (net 4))
 (segment (start 145.732 106.24) (end 145.8 106.172) (width 0.25) (layer "F.Cu") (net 4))
 (segment (start 138.44 101.028522) (end 138.203077 100.791599) (width 0.25) (layer "F.Cu") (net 4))
 (segment (start 154.076923 103.041923) (end 154.076923 105.213449) (width 0.25) (layer "F.Cu") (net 4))
 (segment (start 139.006186 106.718251) (end 139.006186 104.982587) (width 0.25) (layer "F.Cu") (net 4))
 (segment (start 141.402587 108.692587) (end 141.402587 108.258814) (width 0.25) (layer "F.Cu") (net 4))
 (segment (start 144.312996 93.315) (end 146.36 93.315) (width 0.25) (layer "F.Cu") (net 4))
 (segment (start 152.358814 107.718855) (end 150.943855 109.133814) (width 0.25) (layer "F.Cu") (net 4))
 (segment (start 153.8 102.765) (end 154.076923 103.041923) (width 0.25) (layer "F.Cu") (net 4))
 (segment (start 137.753077 103.729478) (end 137.753077 101.715445) (width 0.25) (layer "F.Cu") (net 4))
 (via (at 143.764 111.252) (size 0.8) (drill 0.4) (layers "F.Cu" "B.Cu") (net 4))
 (via (at 144.27 106.24) (size 0.8) (drill 0.4) (layers "F.Cu" "B.Cu") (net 4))
 (segment (start 143.764 106.746) (end 143.764 111.252) (width 0.25) (layer "B.Cu") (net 4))
 (segment (start 144.27 106.24) (end 143.764 106.746) (width 0.25) (layer "B.Cu") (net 4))
 (segment (start 145.140624 93.99) (end 143.58181 95.548814) (width 0.25) (layer "F.Cu") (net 17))
 (segment (start 145.205 93.99) (end 145.140624 93.99) (width 0.25) (layer "F.Cu") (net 17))
 (segment (start 140.873814 96.084356) (end 141.446984 95.511186) (width 0.25) (layer "F.Cu") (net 16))
 (segment (start 140.873814 97.782587) (end 140.873814 96.084356) (width 0.25) (layer "F.Cu") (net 16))
 (segment (start 139.54 100.428522) (end 139.006186 99.894708) (width 0.25) (layer "F.Cu") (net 22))
 (segment (start 139.006186 99.894708) (end 139.006186 98.817413) (width 0.25) (layer "F.Cu") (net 22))
 (segment (start 139.54 101.028522) (end 139.54 100.428522) (width 0.25) (layer "F.Cu") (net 22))
 (segment (start 139.958814 104.432587) (end 139.554669 104.432587) (width 0.25) (layer "F.Cu") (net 21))
 (segment (start 138.44 103.317918) (end 138.44 102.858522) (width 0.25) (layer "F.Cu") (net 21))
 (segment (start 139.554669 104.432587) (end 138.44 103.317918) (width 0.25) (layer "F.Cu") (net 21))
 (segment (start 141.952587 107.306186) (end 140.659959 107.306186) (width 0.25) (layer "F.Cu") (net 3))
 (segment (start 140.659959 107.306186) (end 139.921186 106.567413) (width 0.25) (layer "F.Cu") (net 3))
 (segment (start 143.650623 109.173814) (end 142.987413 109.173814) (width 0.25) (layer "F.Cu") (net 1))
 (segment (start 145.175 108.64) (end 144.184437 108.64) (width 0.25) (layer "F.Cu") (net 1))
 (segment (start 144.184437 108.64) (end 143.650623 109.173814) (width 0.25) (layer "F.Cu") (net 1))
 (segment (start 148.658191 108.181186) (end 147.099377 109.74) (width 0.25) (layer "F.Cu") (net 15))
 (segment (start 147.099377 109.74) (end 147.005 109.74) (width 0.25) (layer "F.Cu") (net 15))
 (segment (start 151.406186 107.605645) (end 150.793017 108.218814) (width 0.25) (layer "F.Cu") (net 20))
 (segment (start 151.406186 105.977413) (end 151.406186 107.605645) (width 0.25) (layer "F.Cu") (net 20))
 (segment (start 152.7 103.365) (end 153.273814 103.938814) (width 0.25) (layer "F.Cu") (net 19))
 (segment (start 152.7 102.765) (end 152.7 103.365) (width 0.25) (layer "F.Cu") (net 19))
 (segment (start 153.273814 103.938814) (end 153.273814 104.942587) (width 0.25) (layer "F.Cu") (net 19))
 (segment (start 153.8 100.746227) (end 153.8 100.935) (width 0.25) (layer "F.Cu") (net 14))
 (segment (start 152.321186 99.267413) (end 153.8 100.746227) (width 0.25) (layer "F.Cu") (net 14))
 (segment (start 150.217413 96.463814) (end 151.690041 96.463814) (width 0.25) (layer "F.Cu") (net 13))
 (segment (start 151.690041 96.463814) (end 152.358814 97.132587) (width 0.25) (layer "F.Cu") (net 13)))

